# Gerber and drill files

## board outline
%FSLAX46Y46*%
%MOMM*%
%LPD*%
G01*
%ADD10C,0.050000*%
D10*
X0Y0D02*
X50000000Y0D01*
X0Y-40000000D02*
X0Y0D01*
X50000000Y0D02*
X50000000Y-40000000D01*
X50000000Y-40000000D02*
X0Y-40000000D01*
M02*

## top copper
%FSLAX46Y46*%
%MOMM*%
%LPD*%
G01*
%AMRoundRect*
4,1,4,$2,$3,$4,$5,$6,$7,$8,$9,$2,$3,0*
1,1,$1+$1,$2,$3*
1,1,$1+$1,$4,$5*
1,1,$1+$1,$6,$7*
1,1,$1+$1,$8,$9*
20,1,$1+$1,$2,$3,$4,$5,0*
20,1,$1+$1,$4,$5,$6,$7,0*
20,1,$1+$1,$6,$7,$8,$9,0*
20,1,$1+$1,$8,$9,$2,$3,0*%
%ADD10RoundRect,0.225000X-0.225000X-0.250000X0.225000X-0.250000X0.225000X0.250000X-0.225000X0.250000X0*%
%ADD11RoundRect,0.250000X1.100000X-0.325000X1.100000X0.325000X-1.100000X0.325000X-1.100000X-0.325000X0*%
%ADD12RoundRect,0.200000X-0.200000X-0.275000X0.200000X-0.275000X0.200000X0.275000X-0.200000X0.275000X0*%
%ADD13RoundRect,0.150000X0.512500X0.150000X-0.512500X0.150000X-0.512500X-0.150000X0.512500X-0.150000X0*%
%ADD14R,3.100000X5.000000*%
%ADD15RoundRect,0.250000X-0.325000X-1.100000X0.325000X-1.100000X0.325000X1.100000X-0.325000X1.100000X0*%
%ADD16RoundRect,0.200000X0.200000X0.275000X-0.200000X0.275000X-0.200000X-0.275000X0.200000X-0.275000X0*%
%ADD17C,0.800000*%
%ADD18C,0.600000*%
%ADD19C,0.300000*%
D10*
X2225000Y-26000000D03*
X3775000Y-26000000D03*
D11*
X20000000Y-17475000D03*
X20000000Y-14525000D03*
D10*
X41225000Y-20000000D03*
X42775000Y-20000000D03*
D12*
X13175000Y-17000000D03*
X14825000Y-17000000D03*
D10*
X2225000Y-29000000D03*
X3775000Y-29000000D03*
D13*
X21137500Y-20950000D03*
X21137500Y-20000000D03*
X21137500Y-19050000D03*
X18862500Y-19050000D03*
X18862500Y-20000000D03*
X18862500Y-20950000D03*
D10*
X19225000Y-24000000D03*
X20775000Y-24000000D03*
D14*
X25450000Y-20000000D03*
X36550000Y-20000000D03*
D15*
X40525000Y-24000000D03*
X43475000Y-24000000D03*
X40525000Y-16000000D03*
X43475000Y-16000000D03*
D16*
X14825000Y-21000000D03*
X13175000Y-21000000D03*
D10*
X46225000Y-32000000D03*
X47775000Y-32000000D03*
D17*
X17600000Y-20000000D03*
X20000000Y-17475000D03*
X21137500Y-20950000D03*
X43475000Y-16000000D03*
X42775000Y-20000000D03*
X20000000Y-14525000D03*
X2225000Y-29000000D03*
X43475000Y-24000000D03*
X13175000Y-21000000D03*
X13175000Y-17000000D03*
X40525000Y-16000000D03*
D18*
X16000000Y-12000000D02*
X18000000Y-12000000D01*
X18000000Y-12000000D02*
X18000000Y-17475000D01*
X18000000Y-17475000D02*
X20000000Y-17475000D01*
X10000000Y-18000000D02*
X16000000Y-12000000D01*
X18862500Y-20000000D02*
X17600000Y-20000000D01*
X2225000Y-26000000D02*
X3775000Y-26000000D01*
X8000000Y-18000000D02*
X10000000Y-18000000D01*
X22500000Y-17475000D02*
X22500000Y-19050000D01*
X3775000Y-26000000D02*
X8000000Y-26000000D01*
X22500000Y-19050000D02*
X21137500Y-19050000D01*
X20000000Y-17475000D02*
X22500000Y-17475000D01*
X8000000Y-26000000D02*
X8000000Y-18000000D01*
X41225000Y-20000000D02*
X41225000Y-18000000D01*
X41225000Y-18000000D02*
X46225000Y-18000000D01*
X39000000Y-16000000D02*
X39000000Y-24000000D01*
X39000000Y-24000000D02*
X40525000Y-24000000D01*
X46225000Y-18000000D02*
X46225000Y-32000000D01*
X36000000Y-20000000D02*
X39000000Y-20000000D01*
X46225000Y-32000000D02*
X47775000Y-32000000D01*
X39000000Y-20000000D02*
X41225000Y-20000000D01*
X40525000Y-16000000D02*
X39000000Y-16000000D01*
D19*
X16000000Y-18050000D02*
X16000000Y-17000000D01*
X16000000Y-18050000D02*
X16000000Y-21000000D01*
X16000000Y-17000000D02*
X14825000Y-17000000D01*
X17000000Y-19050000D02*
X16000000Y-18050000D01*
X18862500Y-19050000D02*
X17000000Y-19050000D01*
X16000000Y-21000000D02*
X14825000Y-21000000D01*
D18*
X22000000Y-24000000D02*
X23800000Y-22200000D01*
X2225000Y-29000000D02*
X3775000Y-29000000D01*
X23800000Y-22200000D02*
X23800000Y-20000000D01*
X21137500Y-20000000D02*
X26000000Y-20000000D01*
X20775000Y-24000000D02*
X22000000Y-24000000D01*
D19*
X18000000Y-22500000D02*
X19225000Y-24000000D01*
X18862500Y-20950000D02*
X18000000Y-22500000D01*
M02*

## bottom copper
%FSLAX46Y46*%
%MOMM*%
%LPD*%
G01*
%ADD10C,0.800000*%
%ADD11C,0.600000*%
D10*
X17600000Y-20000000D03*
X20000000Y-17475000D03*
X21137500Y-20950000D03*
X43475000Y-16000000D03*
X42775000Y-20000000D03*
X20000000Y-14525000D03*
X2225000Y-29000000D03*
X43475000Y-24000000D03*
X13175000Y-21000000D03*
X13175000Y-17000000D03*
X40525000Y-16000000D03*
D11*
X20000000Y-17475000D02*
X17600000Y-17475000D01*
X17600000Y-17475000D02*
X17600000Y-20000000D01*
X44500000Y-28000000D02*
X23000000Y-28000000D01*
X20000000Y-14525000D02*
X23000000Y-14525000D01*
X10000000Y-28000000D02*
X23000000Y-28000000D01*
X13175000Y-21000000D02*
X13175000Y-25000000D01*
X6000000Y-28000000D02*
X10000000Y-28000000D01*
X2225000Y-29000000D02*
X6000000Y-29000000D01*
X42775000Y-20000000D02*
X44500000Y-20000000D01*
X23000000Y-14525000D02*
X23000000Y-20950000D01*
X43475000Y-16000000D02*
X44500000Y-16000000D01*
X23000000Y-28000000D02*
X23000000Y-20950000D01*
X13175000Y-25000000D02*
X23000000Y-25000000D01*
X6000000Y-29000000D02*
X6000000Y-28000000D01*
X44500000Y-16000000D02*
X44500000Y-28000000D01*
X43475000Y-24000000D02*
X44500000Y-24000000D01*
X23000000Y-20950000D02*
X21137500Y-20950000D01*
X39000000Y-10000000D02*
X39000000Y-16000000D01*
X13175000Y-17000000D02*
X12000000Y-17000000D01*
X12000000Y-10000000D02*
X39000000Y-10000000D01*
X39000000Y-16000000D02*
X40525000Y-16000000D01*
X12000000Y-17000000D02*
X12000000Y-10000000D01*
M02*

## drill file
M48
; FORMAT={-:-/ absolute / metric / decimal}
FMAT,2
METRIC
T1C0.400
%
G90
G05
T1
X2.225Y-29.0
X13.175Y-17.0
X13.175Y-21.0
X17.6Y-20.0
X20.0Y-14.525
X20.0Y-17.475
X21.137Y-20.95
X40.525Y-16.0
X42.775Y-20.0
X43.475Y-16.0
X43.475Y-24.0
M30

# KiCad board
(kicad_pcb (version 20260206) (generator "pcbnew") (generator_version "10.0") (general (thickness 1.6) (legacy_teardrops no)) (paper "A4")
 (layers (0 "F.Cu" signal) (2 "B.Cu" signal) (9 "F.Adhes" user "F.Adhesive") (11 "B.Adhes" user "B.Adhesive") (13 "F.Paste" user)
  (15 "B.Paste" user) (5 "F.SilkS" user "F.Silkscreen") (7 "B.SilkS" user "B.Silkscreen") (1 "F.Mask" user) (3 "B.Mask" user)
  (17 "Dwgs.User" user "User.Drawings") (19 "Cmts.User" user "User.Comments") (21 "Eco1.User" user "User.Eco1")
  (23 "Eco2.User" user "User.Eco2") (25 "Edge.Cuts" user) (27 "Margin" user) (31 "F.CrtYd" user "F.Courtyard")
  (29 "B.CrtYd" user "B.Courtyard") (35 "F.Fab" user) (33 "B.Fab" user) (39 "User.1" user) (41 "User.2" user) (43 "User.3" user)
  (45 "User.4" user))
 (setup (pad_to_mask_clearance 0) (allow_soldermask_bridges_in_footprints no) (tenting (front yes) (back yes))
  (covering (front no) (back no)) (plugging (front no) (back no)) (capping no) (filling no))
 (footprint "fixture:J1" (layer "F.Cu") (at 3 26)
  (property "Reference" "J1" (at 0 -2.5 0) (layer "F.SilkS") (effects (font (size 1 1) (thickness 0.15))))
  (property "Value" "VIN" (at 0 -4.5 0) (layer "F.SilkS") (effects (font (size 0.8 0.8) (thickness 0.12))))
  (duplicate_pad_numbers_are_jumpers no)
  (pad "1" smd roundrect (at -0.775 0) (size 0.9 0.95) (layers "F.Cu" "F.Mask" "F.Paste") (roundrect_rratio 0.25) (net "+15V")
   (thermal_bridge_angle 45))
  (pad "2" smd roundrect (at 0.775 0) (size 0.9 0.95) (layers "F.Cu" "F.Mask" "F.Paste") (roundrect_rratio 0.25) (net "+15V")
   (thermal_bridge_angle 45)))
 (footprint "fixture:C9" (layer "F.Cu") (at 20 16 90)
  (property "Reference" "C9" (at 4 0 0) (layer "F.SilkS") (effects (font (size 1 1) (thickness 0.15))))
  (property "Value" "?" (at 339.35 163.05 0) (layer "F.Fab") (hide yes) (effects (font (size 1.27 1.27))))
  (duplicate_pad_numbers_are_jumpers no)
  (pad "1" smd roundrect (at -1.475 0 90) (size 1.15 2.7) (layers "F.Cu" "F.Mask" "F.Paste") (roundrect_rratio 0.217391) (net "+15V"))
  (pad "2" smd roundrect (at 1.475 0 90) (size 1.15 2.7) (layers "F.Cu" "F.Mask" "F.Paste") (roundrect_rratio 0.217391) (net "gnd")))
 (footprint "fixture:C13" (layer "F.Cu") (at 42 20)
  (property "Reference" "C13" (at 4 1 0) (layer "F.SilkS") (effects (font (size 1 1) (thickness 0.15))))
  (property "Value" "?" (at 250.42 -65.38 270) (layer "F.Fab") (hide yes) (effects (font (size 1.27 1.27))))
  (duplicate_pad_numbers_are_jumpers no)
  (pad "1" smd roundrect (at -0.775 0) (size 0.9 0.95) (layers "F.Cu" "F.Mask" "F.Paste") (roundrect_rratio 0.25) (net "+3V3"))
  (pad "2" smd roundrect (at 0.775 0) (size 0.9 0.95) (layers "F.Cu" "F.Mask" "F.Paste") (roundrect_rratio 0.25) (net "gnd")))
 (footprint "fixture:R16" (layer "F.Cu") (at 14 17)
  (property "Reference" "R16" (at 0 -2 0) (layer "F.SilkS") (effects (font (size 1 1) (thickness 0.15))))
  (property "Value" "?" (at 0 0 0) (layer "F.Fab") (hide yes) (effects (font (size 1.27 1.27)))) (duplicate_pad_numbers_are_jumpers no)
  (pad "1" smd roundrect (at -0.825 0) (size 0.8 0.95) (layers "F.Cu" "F.Mask" "F.Paste") (roundrect_rratio 0.25) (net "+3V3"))
  (pad "2" smd roundrect (at 0.825 0) (size 0.8 0.95) (layers "F.Cu" "F.Mask" "F.Paste") (roundrect_rratio 0.25) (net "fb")))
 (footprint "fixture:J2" (layer "F.Cu") (at 3 29)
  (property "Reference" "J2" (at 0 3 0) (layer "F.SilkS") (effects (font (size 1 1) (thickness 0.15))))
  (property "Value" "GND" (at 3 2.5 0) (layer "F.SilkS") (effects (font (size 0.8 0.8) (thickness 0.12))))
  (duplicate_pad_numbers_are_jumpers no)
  (pad "1" smd roundrect (at -0.775 0) (size 0.9 0.95) (layers "F.Cu" "F.Mask" "F.Paste") (roundrect_rratio 0.25) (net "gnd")
   (thermal_bridge_angle 45))
  (pad "2" smd roundrect (at 0.775 0) (size 0.9 0.95) (layers "F.Cu" "F.Mask" "F.Paste") (roundrect_rratio 0.25) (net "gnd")
   (thermal_bridge_angle 45)))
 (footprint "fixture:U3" (layer "F.Cu") (at 20 20 180)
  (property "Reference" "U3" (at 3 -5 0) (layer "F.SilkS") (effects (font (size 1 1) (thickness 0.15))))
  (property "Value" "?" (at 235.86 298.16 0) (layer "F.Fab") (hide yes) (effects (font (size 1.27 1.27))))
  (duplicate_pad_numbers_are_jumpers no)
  (pad "1" smd roundrect (at -1.1375 -0.95 180) (size 1.325 0.6) (layers "F.Cu" "F.Mask" "F.Paste") (roundrect_rratio 0.25) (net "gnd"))
  (pad "2" smd roundrect (at -1.1375 0 180) (size 1.325 0.6) (layers "F.Cu" "F.Mask" "F.Paste") (roundrect_rratio 0.25) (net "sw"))
  (pad "3" smd roundrect (at -1.1375 0.95 180) (size 1.325 0.6) (layers "F.Cu" "F.Mask" "F.Paste") (roundrect_rratio 0.25) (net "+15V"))
  (pad "4" smd roundrect (at 1.1375 0.95 180) (size 1.325 0.6) (layers "F.Cu" "F.Mask" "F.Paste") (roundrect_rratio 0.25) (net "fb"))
  (pad "5" smd roundrect (at 1.1375 0 180) (size 1.325 0.6) (layers "F.Cu" "F.Mask" "F.Paste") (roundrect_rratio 0.25) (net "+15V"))
  (pad "6" smd roundrect (at 1.1375 -0.95 180) (size 1.325 0.6) (layers "F.Cu" "F.Mask" "F.Paste") (roundrect_rratio 0.25) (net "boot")))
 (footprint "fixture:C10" (layer "F.Cu") (at 20 24)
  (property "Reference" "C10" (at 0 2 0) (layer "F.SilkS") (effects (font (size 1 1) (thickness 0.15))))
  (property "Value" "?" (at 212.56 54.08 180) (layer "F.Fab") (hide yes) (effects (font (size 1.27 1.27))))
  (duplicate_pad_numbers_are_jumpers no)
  (pad "1" smd roundrect (at -0.775 0) (size 0.9 0.95) (layers "F.Cu" "F.Mask" "F.Paste") (roundrect_rratio 0.25) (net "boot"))
  (pad "2" smd roundrect (at 0.775 0) (size 0.9 0.95) (layers "F.Cu" "F.Mask" "F.Paste") (roundrect_rratio 0.25) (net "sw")))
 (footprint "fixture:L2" (layer "F.Cu") (at 31 20)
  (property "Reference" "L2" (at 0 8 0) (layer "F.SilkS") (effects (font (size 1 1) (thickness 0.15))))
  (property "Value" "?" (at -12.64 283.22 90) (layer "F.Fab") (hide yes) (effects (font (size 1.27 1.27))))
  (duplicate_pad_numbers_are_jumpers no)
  (pad "1" smd rect (at -5.55 0) (size 3.1 5) (layers "F.Cu" "F.Mask" "F.Paste") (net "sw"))
  (pad "2" smd rect (at 5.55 0) (size 3.1 5) (layers "F.Cu" "F.Mask" "F.Paste") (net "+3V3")))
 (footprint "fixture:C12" (layer "F.Cu") (at 42 24)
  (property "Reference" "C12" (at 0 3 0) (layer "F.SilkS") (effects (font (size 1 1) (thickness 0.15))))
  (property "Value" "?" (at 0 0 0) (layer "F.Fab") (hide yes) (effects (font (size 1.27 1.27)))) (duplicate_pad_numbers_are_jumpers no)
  (pad "1" smd roundrect (at -1.475 0) (size 1.15 2.7) (layers "F.Cu" "F.Mask" "F.Paste") (roundrect_rratio 0.217391) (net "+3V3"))
  (pad "2" smd roundrect (at 1.475 0) (size 1.15 2.7) (layers "F.Cu" "F.Mask" "F.Paste") (roundrect_rratio 0.217391) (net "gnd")))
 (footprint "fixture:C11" (layer "F.Cu") (at 42 16)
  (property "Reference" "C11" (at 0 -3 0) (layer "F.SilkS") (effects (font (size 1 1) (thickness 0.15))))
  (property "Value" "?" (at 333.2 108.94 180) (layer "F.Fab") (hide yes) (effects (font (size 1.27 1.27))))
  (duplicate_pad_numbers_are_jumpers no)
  (pad "1" smd roundrect (at -1.475 0) (size 1.15 2.7) (layers "F.Cu" "F.Mask" "F.Paste") (roundrect_rratio 0.217391) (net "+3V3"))
  (pad "2" smd roundrect (at 1.475 0) (size 1.15 2.7) (layers "F.Cu" "F.Mask" "F.Paste") (roundrect_rratio 0.217391) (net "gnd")))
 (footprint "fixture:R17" (layer "F.Cu") (at 14 21 180)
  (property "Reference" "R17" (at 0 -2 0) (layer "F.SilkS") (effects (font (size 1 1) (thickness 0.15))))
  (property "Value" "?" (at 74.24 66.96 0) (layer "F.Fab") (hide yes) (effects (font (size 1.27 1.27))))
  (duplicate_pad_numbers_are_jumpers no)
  (pad "1" smd roundrect (at -0.825 0 180) (size 0.8 0.95) (layers "F.Cu" "F.Mask" "F.Paste") (roundrect_rratio 0.25) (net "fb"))
  (pad "2" smd roundrect (at 0.825 0 180) (size 0.8 0.95) (layers "F.Cu" "F.Mask" "F.Paste") (roundrect_rratio 0.25) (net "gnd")))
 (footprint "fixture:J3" (layer "F.Cu") (at 47 32)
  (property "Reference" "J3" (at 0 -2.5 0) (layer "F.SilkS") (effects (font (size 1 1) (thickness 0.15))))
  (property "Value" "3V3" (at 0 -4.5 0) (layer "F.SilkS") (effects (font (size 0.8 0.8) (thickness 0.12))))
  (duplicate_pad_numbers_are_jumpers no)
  (pad "1" smd roundrect (at -0.775 0) (size 0.9 0.95) (layers "F.Cu" "F.Mask" "F.Paste") (roundrect_rratio 0.25) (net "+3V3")
   (thermal_bridge_angle 45))
  (pad "2" smd roundrect (at 0.775 0) (size 0.9 0.95) (layers "F.Cu" "F.Mask" "F.Paste") (roundrect_rratio 0.25) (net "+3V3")
   (thermal_bridge_angle 45)))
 (gr_line (start 0 0) (end 50 0) (stroke (width 0.05) (type default)) (layer "Edge.Cuts"))
 (gr_line (start 0 40) (end 0 0) (stroke (width 0.05) (type default)) (layer "Edge.Cuts"))
 (gr_line (start 50 0) (end 50 40) (stroke (width 0.05) (type default)) (layer "Edge.Cuts"))
 (gr_line (start 50 40) (end 0 40) (stroke (width 0.05) (type default)) (layer "Edge.Cuts"))
 (segment (start 16 12) (end 18 12) (width 0.6) (layer "F.Cu") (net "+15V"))
 (segment (start 18 12) (end 18 17.475) (width 0.6) (layer "F.Cu") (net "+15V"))
 (segment (start 18 17.475) (end 20 17.475) (width 0.6) (layer "F.Cu") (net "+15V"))
 (segment (start 10 18) (end 16 12) (width 0.6) (layer "F.Cu") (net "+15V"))
 (segment (start 18.8625 20) (end 17.6 20) (width 0.6) (layer "F.Cu") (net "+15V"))
 (segment (start 2.225 26) (end 3.775 26) (width 0.6) (layer "F.Cu") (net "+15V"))
 (segment (start 8 18) (end 10 18) (width 0.6) (layer "F.Cu") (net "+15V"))
 (segment (start 22.5 17.475) (end 22.5 19.05) (width 0.6) (layer "F.Cu") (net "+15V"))
 (segment (start 3.775 26) (end 8 26) (width 0.6) (layer "F.Cu") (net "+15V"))
 (segment (start 22.5 19.05) (end 21.1375 19.05) (width 0.6) (layer "F.Cu") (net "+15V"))
 (segment (start 20 17.475) (end 22.5 17.475) (width 0.6) (layer "F.Cu") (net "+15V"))
 (segment (start 8 26) (end 8 18) (width 0.6) (layer "F.Cu") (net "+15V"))
 (via (at 17.6 20) (size 0.8) (drill 0.4) (layers "F.Cu" "B.Cu") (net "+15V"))
 (via (at 20 17.475) (size 0.8) (drill 0.4) (layers "F.Cu" "B.Cu") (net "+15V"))
 (segment (start 20 17.475) (end 17.6 17.475) (width 0.6) (layer "B.Cu") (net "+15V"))
 (segment (start 17.6 17.475) (end 17.6 20) (width 0.6) (layer "B.Cu") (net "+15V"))
 (via (at 21.1375 20.95) (size 0.8) (drill 0.4) (layers "F.Cu" "B.Cu") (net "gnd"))
 (via (at 43.475 16) (size 0.8) (drill 0.4) (layers "F.Cu" "B.Cu") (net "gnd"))
 (via (at 42.775 20) (size 0.8) (drill 0.4) (layers "F.Cu" "B.Cu") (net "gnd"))
 (via (at 20 14.525) (size 0.8) (drill 0.4) (layers "F.Cu" "B.Cu") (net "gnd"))
 (via (at 2.225 29) (size 0.8) (drill 0.4) (layers "F.Cu" "B.Cu") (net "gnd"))
 (via (at 43.475 24) (size 0.8) (drill 0.4) (layers "F.Cu" "B.Cu") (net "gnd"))
 (via (at 13.175 21) (size 0.8) (drill 0.4) (layers "F.Cu" "B.Cu") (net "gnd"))
 (segment (start 44.5 28) (end 23 28) (width 0.6) (layer "B.Cu") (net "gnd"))
 (segment (start 20 14.525) (end 23 14.525) (width 0.6) (layer "B.Cu") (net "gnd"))
 (segment (start 10 28) (end 23 28) (width 0.6) (layer "B.Cu") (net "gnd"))
 (segment (start 13.175 21) (end 13.175 25) (width 0.6) (layer "B.Cu") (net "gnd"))
 (segment (start 6 28) (end 10 28) (width 0.6) (layer "B.Cu") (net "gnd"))
 (segment (start 2.225 29) (end 6 29) (width 0.6) (layer "B.Cu") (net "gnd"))
 (segment (start 42.775 20) (end 44.5 20) (width 0.6) (layer "B.Cu") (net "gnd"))
 (segment (start 23 14.525) (end 23 20.95) (width 0.6) (layer "B.Cu") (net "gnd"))
 (segment (start 43.475 16) (end 44.5 16) (width 0.6) (layer "B.Cu") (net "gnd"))
 (segment (start 23 28) (end 23 20.95) (width 0.6) (layer "B.Cu") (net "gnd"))
 (segment (start 13.175 25) (end 23 25) (width 0.6) (layer "B.Cu") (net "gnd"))
 (segment (start 6 29) (end 6 28) (width 0.6) (layer "B.Cu") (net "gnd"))
 (segment (start 44.5 16) (end 44.5 28) (width 0.6) (layer "B.Cu") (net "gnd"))
 (segment (start 43.475 24) (end 44.5 24) (width 0.6) (layer "B.Cu") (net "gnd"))
 (segment (start 23 20.95) (end 21.1375 20.95) (width 0.6) (layer "B.Cu") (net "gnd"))
 (segment (start 41.225 20) (end 41.225 18) (width 0.6) (layer "F.Cu") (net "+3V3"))
 (segment (start 41.225 18) (end 46.225 18) (width 0.6) (layer "F.Cu") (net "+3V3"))
 (segment (start 39 16) (end 39 24) (width 0.6) (layer "F.Cu") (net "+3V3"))
 (segment (start 39 24) (end 40.525 24) (width 0.6) (layer "F.Cu") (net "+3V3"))
 (segment (start 46.225 18) (end 46.225 32) (width 0.6) (layer "F.Cu") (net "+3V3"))
 (segment (start 36 20) (end 39 20) (width 0.6) (layer "F.Cu") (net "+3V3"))
 (segment (start 46.225 32) (end 47.775 32) (width 0.6) (layer "F.Cu") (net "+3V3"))
 (segment (start 39 20) (end 41.225 20) (width 0.6) (layer "F.Cu") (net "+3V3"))
 (segment (start 40.525 16) (end 39 16) (width 0.6) (layer "F.Cu") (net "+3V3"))
 (via (at 13.175 17) (size 0.8) (drill 0.4) (layers "F.Cu" "B.Cu") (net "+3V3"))
 (via (at 40.525 16) (size 0.8) (drill 0.4) (layers "F.Cu" "B.Cu") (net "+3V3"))
 (segment (start 39 10) (end 39 16) (width 0.6) (layer "B.Cu") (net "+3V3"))
 (segment (start 13.175 17) (end 12 17) (width 0.6) (layer "B.Cu") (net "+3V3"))
 (segment (start 12 10) (end 39 10) (width 0.6) (layer "B.Cu") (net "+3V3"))
 (segment (start 39 16) (end 40.525 16) (width 0.6) (layer "B.Cu") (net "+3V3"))
 (segment (start 12 17) (end 12 10) (width 0.6) (layer "B.Cu") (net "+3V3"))
 (segment (start 16 18.05) (end 16 17) (width 0.3) (layer "F.Cu") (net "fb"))
 (segment (start 16 18.05) (end 16 21) (width 0.3) (layer "F.Cu") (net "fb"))
 (segment (start 16 17) (end 14.825 17) (width 0.3) (layer "F.Cu") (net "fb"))
 (segment (start 17 19.05) (end 16 18.05) (width 0.3) (layer "F.Cu") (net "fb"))
 (segment (start 18.8625 19.05) (end 17 19.05) (width 0.3) (layer "F.Cu") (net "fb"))
 (segment (start 16 21) (end 14.825 21) (width 0.3) (layer "F.Cu") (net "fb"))
 (segment (start 22 24) (end 23.8 22.2) (width 0.6) (layer "F.Cu") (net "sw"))
 (segment (start 2.225 29) (end 3.775 29) (width 0.6) (layer "F.Cu") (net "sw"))
 (segment (start 23.8 22.2) (end 23.8 20) (width 0.6) (layer "F.Cu") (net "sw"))
 (segment (start 21.1375 20) (end 26 20) (width 0.6) (layer "F.Cu") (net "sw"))
 (segment (start 20.775 24) (end 22 24) (width 0.6) (layer "F.Cu") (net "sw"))
 (segment (start 18 22.5) (end 19.225 24) (width 0.3) (layer "F.Cu") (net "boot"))
 (segment (start 18.8625 20.95) (end 18 22.5) (width 0.3) (layer "F.Cu") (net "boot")))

